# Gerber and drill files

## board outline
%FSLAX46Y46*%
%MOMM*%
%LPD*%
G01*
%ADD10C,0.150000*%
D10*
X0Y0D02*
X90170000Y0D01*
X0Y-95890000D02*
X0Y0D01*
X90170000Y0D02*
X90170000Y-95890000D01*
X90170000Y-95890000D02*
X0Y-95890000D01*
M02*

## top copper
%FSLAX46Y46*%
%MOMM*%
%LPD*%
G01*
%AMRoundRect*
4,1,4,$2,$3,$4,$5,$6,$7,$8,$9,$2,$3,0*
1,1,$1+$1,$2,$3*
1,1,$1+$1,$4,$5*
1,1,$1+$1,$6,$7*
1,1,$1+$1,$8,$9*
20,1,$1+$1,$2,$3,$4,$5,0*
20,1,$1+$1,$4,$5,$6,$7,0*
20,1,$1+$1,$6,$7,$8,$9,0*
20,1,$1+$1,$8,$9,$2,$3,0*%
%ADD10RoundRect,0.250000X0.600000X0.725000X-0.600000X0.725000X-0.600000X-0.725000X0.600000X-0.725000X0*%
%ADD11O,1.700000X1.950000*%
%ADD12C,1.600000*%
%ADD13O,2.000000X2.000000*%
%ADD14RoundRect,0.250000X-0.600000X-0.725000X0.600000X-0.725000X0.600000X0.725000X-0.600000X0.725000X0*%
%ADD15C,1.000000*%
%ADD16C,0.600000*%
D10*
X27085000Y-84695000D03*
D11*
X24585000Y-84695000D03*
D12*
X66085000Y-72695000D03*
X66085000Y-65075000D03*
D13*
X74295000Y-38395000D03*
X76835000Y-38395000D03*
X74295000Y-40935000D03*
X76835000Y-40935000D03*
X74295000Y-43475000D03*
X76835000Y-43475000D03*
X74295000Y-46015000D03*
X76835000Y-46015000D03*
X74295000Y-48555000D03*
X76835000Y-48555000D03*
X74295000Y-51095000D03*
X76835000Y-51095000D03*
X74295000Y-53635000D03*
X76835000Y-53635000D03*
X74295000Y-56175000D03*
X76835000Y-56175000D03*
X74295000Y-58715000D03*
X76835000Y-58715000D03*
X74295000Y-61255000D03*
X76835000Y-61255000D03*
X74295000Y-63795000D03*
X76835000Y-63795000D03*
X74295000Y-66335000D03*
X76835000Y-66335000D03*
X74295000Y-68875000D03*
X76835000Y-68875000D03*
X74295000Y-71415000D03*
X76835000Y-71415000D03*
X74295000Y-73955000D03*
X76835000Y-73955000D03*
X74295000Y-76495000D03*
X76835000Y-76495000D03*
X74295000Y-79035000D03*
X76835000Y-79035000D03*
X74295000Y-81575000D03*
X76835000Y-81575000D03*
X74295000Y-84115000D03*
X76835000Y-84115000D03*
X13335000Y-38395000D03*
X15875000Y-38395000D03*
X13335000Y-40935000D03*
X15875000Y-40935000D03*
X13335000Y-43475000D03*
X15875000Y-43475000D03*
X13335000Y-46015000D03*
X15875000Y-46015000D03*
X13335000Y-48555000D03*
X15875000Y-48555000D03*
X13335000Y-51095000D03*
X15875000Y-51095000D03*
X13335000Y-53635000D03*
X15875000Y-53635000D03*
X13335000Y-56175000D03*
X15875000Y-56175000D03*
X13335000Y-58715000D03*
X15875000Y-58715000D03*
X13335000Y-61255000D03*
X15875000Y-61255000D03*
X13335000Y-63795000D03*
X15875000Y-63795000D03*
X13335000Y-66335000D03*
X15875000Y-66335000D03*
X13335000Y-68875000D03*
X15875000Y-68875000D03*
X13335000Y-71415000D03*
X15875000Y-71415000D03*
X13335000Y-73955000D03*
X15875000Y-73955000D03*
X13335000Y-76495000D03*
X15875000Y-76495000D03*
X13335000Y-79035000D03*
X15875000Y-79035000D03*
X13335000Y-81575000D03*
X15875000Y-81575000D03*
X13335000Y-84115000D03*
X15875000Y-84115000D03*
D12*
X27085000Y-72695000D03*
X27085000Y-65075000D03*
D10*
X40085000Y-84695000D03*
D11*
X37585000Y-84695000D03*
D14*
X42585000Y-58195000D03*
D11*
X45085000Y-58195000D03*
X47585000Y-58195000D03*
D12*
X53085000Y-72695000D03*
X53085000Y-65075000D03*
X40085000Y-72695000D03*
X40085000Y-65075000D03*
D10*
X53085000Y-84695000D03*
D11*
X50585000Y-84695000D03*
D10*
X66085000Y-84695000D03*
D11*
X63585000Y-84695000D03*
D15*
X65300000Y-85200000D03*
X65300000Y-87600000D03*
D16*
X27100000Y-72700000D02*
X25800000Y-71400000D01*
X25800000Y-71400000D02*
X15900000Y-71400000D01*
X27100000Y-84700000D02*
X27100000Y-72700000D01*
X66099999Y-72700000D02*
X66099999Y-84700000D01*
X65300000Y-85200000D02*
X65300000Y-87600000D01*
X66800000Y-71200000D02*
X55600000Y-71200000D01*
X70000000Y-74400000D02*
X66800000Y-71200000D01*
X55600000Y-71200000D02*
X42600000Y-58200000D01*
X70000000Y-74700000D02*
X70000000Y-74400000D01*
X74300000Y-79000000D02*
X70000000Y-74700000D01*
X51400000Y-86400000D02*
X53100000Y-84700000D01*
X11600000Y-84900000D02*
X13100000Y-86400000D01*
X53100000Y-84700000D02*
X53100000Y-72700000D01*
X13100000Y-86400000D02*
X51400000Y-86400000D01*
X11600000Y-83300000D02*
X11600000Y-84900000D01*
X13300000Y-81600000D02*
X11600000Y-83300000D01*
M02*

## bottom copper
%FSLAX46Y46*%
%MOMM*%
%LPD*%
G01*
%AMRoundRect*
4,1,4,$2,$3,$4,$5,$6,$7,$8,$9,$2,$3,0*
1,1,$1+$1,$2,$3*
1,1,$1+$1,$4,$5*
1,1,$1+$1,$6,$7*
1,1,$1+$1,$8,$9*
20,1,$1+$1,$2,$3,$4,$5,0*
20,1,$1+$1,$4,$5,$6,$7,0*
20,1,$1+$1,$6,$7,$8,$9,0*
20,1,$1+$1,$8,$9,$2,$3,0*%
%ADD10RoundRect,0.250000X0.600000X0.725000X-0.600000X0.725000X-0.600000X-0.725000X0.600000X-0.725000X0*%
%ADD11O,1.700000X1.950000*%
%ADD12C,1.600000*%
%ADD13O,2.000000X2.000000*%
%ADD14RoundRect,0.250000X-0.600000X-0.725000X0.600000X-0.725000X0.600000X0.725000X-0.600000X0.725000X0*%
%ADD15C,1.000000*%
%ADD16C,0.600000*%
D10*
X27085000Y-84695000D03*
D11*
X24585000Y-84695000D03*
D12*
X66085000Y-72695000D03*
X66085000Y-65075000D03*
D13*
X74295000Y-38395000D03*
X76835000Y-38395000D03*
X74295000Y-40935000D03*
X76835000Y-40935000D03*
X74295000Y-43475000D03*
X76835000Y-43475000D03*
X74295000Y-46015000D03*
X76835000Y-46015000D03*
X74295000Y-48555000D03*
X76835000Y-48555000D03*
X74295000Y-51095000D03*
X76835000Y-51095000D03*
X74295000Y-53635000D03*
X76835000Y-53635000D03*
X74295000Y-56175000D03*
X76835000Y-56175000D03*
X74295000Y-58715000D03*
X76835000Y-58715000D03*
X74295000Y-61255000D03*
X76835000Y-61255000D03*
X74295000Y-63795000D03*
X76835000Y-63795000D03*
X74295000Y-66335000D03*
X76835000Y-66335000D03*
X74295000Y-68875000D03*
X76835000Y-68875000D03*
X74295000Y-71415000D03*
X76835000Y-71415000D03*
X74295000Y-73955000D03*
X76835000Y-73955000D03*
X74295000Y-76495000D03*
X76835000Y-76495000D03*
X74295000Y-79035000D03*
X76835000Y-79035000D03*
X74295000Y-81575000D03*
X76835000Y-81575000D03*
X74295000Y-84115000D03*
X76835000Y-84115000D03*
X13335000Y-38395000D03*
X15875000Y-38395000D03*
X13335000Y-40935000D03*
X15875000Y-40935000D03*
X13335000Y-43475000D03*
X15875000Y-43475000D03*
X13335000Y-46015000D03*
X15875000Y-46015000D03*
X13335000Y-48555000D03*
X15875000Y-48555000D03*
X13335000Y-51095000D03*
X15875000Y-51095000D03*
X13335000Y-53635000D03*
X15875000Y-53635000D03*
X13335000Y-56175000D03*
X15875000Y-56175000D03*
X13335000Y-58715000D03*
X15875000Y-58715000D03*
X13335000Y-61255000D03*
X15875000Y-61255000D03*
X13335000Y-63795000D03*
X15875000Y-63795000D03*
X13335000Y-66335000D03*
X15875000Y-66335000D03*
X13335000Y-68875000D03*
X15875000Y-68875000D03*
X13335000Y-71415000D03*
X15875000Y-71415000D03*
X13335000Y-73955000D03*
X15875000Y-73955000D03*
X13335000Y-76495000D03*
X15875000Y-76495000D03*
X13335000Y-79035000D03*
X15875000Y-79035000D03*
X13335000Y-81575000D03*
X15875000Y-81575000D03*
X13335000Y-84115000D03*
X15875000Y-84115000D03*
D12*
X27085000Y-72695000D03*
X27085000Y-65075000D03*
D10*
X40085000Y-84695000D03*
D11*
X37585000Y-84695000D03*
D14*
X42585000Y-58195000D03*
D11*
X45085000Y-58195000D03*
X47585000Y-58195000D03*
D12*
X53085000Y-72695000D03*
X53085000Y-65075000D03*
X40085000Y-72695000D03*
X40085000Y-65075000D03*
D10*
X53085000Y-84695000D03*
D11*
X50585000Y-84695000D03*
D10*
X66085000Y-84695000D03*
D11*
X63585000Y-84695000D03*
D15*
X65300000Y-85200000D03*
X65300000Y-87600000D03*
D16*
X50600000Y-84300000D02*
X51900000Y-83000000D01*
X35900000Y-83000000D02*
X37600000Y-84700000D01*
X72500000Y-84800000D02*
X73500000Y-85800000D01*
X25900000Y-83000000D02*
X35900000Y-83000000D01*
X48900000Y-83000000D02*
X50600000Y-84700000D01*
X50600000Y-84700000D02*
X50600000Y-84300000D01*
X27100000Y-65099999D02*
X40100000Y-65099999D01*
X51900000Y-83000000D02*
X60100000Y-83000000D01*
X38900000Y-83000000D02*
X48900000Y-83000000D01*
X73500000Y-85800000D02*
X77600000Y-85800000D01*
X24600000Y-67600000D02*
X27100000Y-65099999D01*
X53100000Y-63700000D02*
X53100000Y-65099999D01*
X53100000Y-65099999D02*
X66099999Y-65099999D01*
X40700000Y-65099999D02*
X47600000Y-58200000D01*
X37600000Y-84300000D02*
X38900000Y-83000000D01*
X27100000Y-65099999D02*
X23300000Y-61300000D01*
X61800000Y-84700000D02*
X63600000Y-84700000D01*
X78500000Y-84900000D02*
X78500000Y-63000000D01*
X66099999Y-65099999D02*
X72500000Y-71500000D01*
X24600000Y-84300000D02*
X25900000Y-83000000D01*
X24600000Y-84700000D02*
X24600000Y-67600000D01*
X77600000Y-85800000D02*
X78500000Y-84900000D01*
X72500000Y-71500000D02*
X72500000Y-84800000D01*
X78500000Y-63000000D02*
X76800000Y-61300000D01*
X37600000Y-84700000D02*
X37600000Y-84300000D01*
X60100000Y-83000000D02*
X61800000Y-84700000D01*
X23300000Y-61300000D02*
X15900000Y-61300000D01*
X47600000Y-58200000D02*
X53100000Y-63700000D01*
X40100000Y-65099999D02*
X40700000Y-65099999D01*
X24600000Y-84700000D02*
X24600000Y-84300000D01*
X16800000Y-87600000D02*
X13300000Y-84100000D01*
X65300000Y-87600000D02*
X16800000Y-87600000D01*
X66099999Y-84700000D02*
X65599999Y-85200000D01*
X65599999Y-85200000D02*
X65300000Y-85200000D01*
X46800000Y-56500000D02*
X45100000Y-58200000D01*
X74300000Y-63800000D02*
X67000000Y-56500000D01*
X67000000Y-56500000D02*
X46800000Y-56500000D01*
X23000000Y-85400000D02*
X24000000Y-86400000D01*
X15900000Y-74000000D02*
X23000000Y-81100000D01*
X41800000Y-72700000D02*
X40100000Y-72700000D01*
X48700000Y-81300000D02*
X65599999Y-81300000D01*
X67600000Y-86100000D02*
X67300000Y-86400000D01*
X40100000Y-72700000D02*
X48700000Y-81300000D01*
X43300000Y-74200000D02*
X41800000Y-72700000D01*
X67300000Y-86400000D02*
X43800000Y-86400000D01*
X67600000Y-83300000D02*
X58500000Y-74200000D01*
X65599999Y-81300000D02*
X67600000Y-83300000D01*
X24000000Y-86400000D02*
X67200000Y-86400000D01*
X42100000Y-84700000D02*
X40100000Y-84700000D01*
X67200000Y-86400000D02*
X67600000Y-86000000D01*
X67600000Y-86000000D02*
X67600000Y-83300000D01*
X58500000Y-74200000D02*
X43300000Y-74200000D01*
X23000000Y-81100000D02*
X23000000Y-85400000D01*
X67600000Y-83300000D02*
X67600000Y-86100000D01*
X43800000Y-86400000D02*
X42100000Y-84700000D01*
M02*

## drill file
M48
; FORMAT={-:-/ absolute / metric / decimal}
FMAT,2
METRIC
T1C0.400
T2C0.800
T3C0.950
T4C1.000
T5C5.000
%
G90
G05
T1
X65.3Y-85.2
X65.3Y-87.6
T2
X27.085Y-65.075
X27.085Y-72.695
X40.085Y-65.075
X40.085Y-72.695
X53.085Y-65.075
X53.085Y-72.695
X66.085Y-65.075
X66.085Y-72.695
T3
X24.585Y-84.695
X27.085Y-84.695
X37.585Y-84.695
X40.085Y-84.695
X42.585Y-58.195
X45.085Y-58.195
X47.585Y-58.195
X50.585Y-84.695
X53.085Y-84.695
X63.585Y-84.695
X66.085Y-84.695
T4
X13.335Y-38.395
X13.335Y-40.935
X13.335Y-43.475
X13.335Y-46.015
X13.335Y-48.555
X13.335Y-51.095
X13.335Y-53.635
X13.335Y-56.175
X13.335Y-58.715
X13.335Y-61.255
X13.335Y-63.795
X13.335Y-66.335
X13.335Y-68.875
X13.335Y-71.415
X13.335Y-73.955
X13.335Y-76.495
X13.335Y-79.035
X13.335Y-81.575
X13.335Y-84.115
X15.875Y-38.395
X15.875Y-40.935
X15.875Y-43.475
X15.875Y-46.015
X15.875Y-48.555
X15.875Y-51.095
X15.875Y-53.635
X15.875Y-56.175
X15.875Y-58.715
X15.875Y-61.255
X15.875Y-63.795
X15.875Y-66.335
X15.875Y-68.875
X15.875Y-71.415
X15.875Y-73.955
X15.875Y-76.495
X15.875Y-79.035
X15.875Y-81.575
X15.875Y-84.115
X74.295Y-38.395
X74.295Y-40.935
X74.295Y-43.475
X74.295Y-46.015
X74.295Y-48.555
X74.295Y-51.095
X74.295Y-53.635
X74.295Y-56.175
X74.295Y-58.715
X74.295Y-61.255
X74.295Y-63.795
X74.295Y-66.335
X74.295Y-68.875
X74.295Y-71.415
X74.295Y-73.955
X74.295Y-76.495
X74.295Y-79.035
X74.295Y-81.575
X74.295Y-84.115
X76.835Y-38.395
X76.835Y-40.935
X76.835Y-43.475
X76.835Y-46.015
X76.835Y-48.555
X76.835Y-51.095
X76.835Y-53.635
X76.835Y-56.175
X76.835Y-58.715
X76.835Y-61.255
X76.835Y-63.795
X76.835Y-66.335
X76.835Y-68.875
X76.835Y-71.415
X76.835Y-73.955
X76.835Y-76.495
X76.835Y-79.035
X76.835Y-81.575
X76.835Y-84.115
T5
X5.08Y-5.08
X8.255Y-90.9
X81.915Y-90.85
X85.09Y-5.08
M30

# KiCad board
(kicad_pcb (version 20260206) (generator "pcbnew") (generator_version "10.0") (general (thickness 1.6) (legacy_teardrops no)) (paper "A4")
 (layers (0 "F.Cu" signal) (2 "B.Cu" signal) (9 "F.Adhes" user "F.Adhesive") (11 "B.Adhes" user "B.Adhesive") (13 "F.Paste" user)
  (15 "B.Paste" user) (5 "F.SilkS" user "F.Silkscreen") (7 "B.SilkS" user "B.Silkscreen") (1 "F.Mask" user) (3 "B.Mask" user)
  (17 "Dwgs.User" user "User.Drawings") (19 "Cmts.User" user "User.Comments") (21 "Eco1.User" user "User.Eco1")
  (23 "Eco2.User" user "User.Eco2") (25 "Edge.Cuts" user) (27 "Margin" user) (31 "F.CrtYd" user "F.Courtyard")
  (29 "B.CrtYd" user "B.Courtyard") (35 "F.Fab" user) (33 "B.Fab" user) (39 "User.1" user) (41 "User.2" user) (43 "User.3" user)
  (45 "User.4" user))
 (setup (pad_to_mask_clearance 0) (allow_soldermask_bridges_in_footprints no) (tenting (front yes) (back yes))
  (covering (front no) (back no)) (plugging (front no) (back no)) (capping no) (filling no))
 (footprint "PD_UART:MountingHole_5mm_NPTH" (layer "F.Cu") (at 8.255 90.9)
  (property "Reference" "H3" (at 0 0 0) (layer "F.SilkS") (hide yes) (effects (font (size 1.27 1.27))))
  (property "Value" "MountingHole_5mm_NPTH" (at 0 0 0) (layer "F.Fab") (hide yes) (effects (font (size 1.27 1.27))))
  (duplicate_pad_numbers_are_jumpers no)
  (pad "" np_thru_hole circle (at 0 0) (size 5 5) (drill 5) (layers "*.Cu")))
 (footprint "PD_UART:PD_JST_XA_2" (layer "F.Cu") (at 27.085 84.695 180)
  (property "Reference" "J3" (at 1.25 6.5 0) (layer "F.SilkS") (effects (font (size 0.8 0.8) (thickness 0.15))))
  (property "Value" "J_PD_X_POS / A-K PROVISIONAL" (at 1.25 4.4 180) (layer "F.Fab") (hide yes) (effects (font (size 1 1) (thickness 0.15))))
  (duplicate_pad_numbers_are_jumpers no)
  (pad "1" thru_hole roundrect (at 0 0 180) (size 1.7 1.95) (drill 0.95) (layers "*.Cu") (remove_unused_layers no)
   (roundrect_rratio 0.147059) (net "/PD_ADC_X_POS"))
  (pad "2" thru_hole oval (at 2.5 0 180) (size 1.7 1.95) (drill 0.95) (layers "*.Cu") (remove_unused_layers no) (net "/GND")))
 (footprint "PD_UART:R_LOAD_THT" (layer "F.Cu") (at 66.085 72.695 90)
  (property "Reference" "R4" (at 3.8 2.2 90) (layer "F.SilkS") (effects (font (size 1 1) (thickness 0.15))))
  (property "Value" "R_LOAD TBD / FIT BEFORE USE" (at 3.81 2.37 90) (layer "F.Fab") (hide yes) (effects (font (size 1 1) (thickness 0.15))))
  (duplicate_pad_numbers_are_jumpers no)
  (pad "1" thru_hole circle (at 0 0 90) (size 1.6 1.6) (drill 0.8) (layers "*.Cu") (remove_unused_layers no) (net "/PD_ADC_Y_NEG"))
  (pad "2" thru_hole circle (at 7.62 0 90) (size 1.6 1.6) (drill 0.8) (layers "*.Cu") (remove_unused_layers no) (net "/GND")))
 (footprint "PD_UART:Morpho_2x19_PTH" (layer "F.Cu") (at 74.295 38.395)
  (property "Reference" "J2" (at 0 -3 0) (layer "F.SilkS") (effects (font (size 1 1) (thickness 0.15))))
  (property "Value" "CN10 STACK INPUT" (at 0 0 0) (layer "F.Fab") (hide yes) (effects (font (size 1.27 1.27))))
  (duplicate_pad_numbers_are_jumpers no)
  (pad "1" thru_hole oval (at 0 0) (size 2 2) (drill 1) (layers "*.Cu") (remove_unused_layers no) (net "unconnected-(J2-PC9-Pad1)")
   (thermal_bridge_angle 45))
  (pad "2" thru_hole oval (at 2.54 0) (size 2 2) (drill 1) (layers "*.Cu") (remove_unused_layers no) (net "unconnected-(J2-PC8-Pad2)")
   (thermal_bridge_angle 45))
  (pad "3" thru_hole oval (at 0 2.54) (size 2 2) (drill 1) (layers "*.Cu") (remove_unused_layers no) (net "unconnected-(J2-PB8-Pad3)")
   (thermal_bridge_angle 45))
  (pad "4" thru_hole oval (at 2.54 2.54) (size 2 2) (drill 1) (layers "*.Cu") (remove_unused_layers no) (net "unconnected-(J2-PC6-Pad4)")
   (thermal_bridge_angle 45))
  (pad "5" thru_hole oval (at 0 5.08) (size 2 2) (drill 1) (layers "*.Cu") (remove_unused_layers no) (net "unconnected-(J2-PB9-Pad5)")
   (thermal_bridge_angle 45))
  (pad "6" thru_hole oval (at 2.54 5.08) (size 2 2) (drill 1) (layers "*.Cu") (remove_unused_layers no) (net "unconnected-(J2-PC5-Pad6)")
   (thermal_bridge_angle 45))
  (pad "7" thru_hole oval (at 0 7.62) (size 2 2) (drill 1) (layers "*.Cu") (remove_unused_layers no) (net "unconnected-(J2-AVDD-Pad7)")
   (thermal_bridge_angle 45))
  (pad "8" thru_hole oval (at 2.54 7.62) (size 2 2) (drill 1) (layers "*.Cu") (remove_unused_layers no) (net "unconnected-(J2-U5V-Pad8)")
   (thermal_bridge_angle 45))
  (pad "9" thru_hole oval (at 0 10.16) (size 2 2) (drill 1) (layers "*.Cu") (remove_unused_layers no) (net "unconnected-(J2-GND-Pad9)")
   (thermal_bridge_angle 45))
  (pad "10" thru_hole oval (at 2.54 10.16) (size 2 2) (drill 1) (layers "*.Cu") (remove_unused_layers no) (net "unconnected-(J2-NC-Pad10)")
   (thermal_bridge_angle 45))
  (pad "11" thru_hole oval (at 0 12.7) (size 2 2) (drill 1) (layers "*.Cu") (remove_unused_layers no) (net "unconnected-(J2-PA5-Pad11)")
   (thermal_bridge_angle 45))
  (pad "12" thru_hole oval (at 2.54 12.7) (size 2 2) (drill 1) (layers "*.Cu") (remove_unused_layers no) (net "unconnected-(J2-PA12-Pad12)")
   (thermal_bridge_angle 45))
  (pad "13" thru_hole oval (at 0 15.24) (size 2 2) (drill 1) (layers "*.Cu") (remove_unused_layers no) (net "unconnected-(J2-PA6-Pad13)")
   (thermal_bridge_angle 45))
  (pad "14" thru_hole oval (at 2.54 15.24) (size 2 2) (drill 1) (layers "*.Cu") (remove_unused_layers no)
   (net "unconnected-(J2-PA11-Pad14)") (thermal_bridge_angle 45))
  (pad "15" thru_hole oval (at 0 17.78) (size 2 2) (drill 1) (layers "*.Cu") (remove_unused_layers no) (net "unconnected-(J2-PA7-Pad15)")
   (thermal_bridge_angle 45))
  (pad "16" thru_hole oval (at 2.54 17.78) (size 2 2) (drill 1) (layers "*.Cu") (remove_unused_layers no)
   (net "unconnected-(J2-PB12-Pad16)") (thermal_bridge_angle 45))
  (pad "17" thru_hole oval (at 0 20.32) (size 2 2) (drill 1) (layers "*.Cu") (remove_unused_layers no) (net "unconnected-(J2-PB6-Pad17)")
   (thermal_bridge_angle 45))
  (pad "18" thru_hole oval (at 2.54 20.32) (size 2 2) (drill 1) (layers "*.Cu") (remove_unused_layers no)
   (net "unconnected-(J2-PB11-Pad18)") (thermal_bridge_angle 45))
  (pad "19" thru_hole oval (at 0 22.86) (size 2 2) (drill 1) (layers "*.Cu") (remove_unused_layers no) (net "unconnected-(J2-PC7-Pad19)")
   (thermal_bridge_angle 45))
  (pad "20" thru_hole oval (at 2.54 22.86) (size 2 2) (drill 1) (layers "*.Cu") (remove_unused_layers no) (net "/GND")
   (thermal_bridge_angle 45))
  (pad "21" thru_hole oval (at 0 25.4) (size 2 2) (drill 1) (layers "*.Cu") (remove_unused_layers no) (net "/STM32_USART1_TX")
   (thermal_bridge_angle 45))
  (pad "22" thru_hole oval (at 2.54 25.4) (size 2 2) (drill 1) (layers "*.Cu") (remove_unused_layers no) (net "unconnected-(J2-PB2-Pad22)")
   (thermal_bridge_angle 45))
  (pad "23" thru_hole oval (at 0 27.94) (size 2 2) (drill 1) (layers "*.Cu") (remove_unused_layers no) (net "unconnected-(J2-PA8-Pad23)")
   (thermal_bridge_angle 45))
  (pad "24" thru_hole oval (at 2.54 27.94) (size 2 2) (drill 1) (layers "*.Cu") (remove_unused_layers no) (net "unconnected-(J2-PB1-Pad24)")
   (thermal_bridge_angle 45))
  (pad "25" thru_hole oval (at 0 30.48) (size 2 2) (drill 1) (layers "*.Cu") (remove_unused_layers no) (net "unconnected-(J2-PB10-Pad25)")
   (thermal_bridge_angle 45))
  (pad "26" thru_hole oval (at 2.54 30.48) (size 2 2) (drill 1) (layers "*.Cu") (remove_unused_layers no)
   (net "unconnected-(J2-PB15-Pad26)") (thermal_bridge_angle 45))
  (pad "27" thru_hole oval (at 0 33.02) (size 2 2) (drill 1) (layers "*.Cu") (remove_unused_layers no) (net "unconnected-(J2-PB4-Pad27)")
   (thermal_bridge_angle 45))
  (pad "28" thru_hole oval (at 2.54 33.02) (size 2 2) (drill 1) (layers "*.Cu") (remove_unused_layers no)
   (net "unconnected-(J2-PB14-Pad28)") (thermal_bridge_angle 45))
  (pad "29" thru_hole oval (at 0 35.56) (size 2 2) (drill 1) (layers "*.Cu") (remove_unused_layers no) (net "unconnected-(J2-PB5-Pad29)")
   (thermal_bridge_angle 45))
  (pad "30" thru_hole oval (at 2.54 35.56) (size 2 2) (drill 1) (layers "*.Cu") (remove_unused_layers no)
   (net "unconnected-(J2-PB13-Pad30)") (thermal_bridge_angle 45))
  (pad "31" thru_hole oval (at 0 38.1) (size 2 2) (drill 1) (layers "*.Cu") (remove_unused_layers no) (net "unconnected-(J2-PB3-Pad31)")
   (thermal_bridge_angle 45))
  (pad "32" thru_hole oval (at 2.54 38.1) (size 2 2) (drill 1) (layers "*.Cu") (remove_unused_layers no) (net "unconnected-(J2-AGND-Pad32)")
   (thermal_bridge_angle 45))
  (pad "33" thru_hole oval (at 0 40.64) (size 2 2) (drill 1) (layers "*.Cu") (remove_unused_layers no) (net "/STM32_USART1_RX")
   (thermal_bridge_angle 45))
  (pad "34" thru_hole oval (at 2.54 40.64) (size 2 2) (drill 1) (layers "*.Cu") (remove_unused_layers no) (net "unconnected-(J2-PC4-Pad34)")
   (thermal_bridge_angle 45))
  (pad "35" thru_hole oval (at 0 43.18) (size 2 2) (drill 1) (layers "*.Cu") (remove_unused_layers no) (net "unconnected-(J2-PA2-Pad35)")
   (thermal_bridge_angle 45))
  (pad "36" thru_hole oval (at 2.54 43.18) (size 2 2) (drill 1) (layers "*.Cu") (remove_unused_layers no) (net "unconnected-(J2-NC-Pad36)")
   (thermal_bridge_angle 45))
  (pad "37" thru_hole oval (at 0 45.72) (size 2 2) (drill 1) (layers "*.Cu") (remove_unused_layers no) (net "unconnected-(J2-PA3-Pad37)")
   (thermal_bridge_angle 45))
  (pad "38" thru_hole oval (at 2.54 45.72) (size 2 2) (drill 1) (layers "*.Cu") (remove_unused_layers no) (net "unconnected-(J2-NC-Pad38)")
   (thermal_bridge_angle 45)))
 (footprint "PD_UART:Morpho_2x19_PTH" (layer "F.Cu") (at 13.335 38.395)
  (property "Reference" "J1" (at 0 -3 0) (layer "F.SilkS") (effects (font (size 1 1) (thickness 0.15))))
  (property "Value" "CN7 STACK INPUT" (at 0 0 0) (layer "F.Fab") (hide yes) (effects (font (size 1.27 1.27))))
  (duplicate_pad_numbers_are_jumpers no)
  (pad "1" thru_hole oval (at 0 0) (size 2 2) (drill 1) (layers "*.Cu") (remove_unused_layers no) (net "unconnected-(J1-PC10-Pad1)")
   (thermal_bridge_angle 45))
  (pad "2" thru_hole oval (at 2.54 0) (size 2 2) (drill 1) (layers "*.Cu") (remove_unused_layers no) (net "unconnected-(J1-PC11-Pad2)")
   (thermal_bridge_angle 45))
  (pad "3" thru_hole oval (at 0 2.54) (size 2 2) (drill 1) (layers "*.Cu") (remove_unused_layers no) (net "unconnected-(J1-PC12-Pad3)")
   (thermal_bridge_angle 45))
  (pad "4" thru_hole oval (at 2.54 2.54) (size 2 2) (drill 1) (layers "*.Cu") (remove_unused_layers no) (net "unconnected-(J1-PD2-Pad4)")
   (thermal_bridge_angle 45))
  (pad "5" thru_hole oval (at 0 5.08) (size 2 2) (drill 1) (layers "*.Cu") (remove_unused_layers no) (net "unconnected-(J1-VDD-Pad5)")
   (thermal_bridge_angle 45))
  (pad "6" thru_hole oval (at 2.54 5.08) (size 2 2) (drill 1) (layers "*.Cu") (remove_unused_layers no) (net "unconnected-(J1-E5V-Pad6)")
   (thermal_bridge_angle 45))
  (pad "7" thru_hole oval (at 0 7.62) (size 2 2) (drill 1) (layers "*.Cu") (remove_unused_layers no) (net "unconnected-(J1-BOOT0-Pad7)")
   (thermal_bridge_angle 45))
  (pad "8" thru_hole oval (at 2.54 7.62) (size 2 2) (drill 1) (layers "*.Cu") (remove_unused_layers no) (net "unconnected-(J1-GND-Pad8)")
   (thermal_bridge_angle 45))
  (pad "9" thru_hole oval (at 0 10.16) (size 2 2) (drill 1) (layers "*.Cu") (remove_unused_layers no) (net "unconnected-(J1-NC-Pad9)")
   (thermal_bridge_angle 45))
  (pad "10" thru_hole oval (at 2.54 10.16) (size 2 2) (drill 1) (layers "*.Cu") (remove_unused_layers no) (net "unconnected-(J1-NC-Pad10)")
   (thermal_bridge_angle 45))
  (pad "11" thru_hole oval (at 0 12.7) (size 2 2) (drill 1) (layers "*.Cu") (remove_unused_layers no) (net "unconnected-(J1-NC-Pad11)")
   (thermal_bridge_angle 45))
  (pad "12" thru_hole oval (at 2.54 12.7) (size 2 2) (drill 1) (layers "*.Cu") (remove_unused_layers no)
   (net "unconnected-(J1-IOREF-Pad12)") (thermal_bridge_angle 45))
  (pad "13" thru_hole oval (at 0 15.24) (size 2 2) (drill 1) (layers "*.Cu") (remove_unused_layers no) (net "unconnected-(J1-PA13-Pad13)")
   (thermal_bridge_angle 45))
  (pad "14" thru_hole oval (at 2.54 15.24) (size 2 2) (drill 1) (layers "*.Cu") (remove_unused_layers no)
   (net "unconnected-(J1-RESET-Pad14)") (thermal_bridge_angle 45))
  (pad "15" thru_hole oval (at 0 17.78) (size 2 2) (drill 1) (layers "*.Cu") (remove_unused_layers no) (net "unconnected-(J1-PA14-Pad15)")
   (thermal_bridge_angle 45))
  (pad "16" thru_hole oval (at 2.54 17.78) (size 2 2) (drill 1) (layers "*.Cu") (remove_unused_layers no) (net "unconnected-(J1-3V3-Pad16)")
   (thermal_bridge_angle 45))
  (pad "17" thru_hole oval (at 0 20.32) (size 2 2) (drill 1) (layers "*.Cu") (remove_unused_layers no) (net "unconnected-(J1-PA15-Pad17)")
   (thermal_bridge_angle 45))
  (pad "18" thru_hole oval (at 2.54 20.32) (size 2 2) (drill 1) (layers "*.Cu") (remove_unused_layers no) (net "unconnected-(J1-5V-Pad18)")
   (thermal_bridge_angle 45))
  (pad "19" thru_hole oval (at 0 22.86) (size 2 2) (drill 1) (layers "*.Cu") (remove_unused_layers no) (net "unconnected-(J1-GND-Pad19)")
   (thermal_bridge_angle 45))
  (pad "20" thru_hole oval (at 2.54 22.86) (size 2 2) (drill 1) (layers "*.Cu") (remove_unused_layers no) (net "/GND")
   (thermal_bridge_angle 45))
  (pad "21" thru_hole oval (at 0 25.4) (size 2 2) (drill 1) (layers "*.Cu") (remove_unused_layers no) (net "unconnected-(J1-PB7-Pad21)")
   (thermal_bridge_angle 45))
  (pad "22" thru_hole oval (at 2.54 25.4) (size 2 2) (drill 1) (layers "*.Cu") (remove_unused_layers no) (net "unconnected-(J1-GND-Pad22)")
   (thermal_bridge_angle 45))
  (pad "23" thru_hole oval (at 0 27.94) (size 2 2) (drill 1) (layers "*.Cu") (remove_unused_layers no) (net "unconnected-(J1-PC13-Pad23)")
   (thermal_bridge_angle 45))
  (pad "24" thru_hole oval (at 2.54 27.94) (size 2 2) (drill 1) (layers "*.Cu") (remove_unused_layers no) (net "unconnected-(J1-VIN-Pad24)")
   (thermal_bridge_angle 45))
  (pad "25" thru_hole oval (at 0 30.48) (size 2 2) (drill 1) (layers "*.Cu") (remove_unused_layers no) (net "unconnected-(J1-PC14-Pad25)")
   (thermal_bridge_angle 45))
  (pad "26" thru_hole oval (at 2.54 30.48) (size 2 2) (drill 1) (layers "*.Cu") (remove_unused_layers no) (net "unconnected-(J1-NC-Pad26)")
   (thermal_bridge_angle 45))
  (pad "27" thru_hole oval (at 0 33.02) (size 2 2) (drill 1) (layers "*.Cu") (remove_unused_layers no) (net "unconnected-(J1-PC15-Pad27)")
   (thermal_bridge_angle 45))
  (pad "28" thru_hole oval (at 2.54 33.02) (size 2 2) (drill 1) (layers "*.Cu") (remove_unused_layers no) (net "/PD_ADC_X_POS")
   (thermal_bridge_angle 45))
  (pad "29" thru_hole oval (at 0 35.56) (size 2 2) (drill 1) (layers "*.Cu") (remove_unused_layers no) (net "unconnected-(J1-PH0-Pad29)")
   (thermal_bridge_angle 45))
  (pad "30" thru_hole oval (at 2.54 35.56) (size 2 2) (drill 1) (layers "*.Cu") (remove_unused_layers no) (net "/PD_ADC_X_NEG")
   (thermal_bridge_angle 45))
  (pad "31" thru_hole oval (at 0 38.1) (size 2 2) (drill 1) (layers "*.Cu") (remove_unused_layers no) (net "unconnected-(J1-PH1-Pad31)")
   (thermal_bridge_angle 45))
  (pad "32" thru_hole oval (at 2.54 38.1) (size 2 2) (drill 1) (layers "*.Cu") (remove_unused_layers no) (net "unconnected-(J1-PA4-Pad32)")
   (thermal_bridge_angle 45))
  (pad "33" thru_hole oval (at 0 40.64) (size 2 2) (drill 1) (layers "*.Cu") (remove_unused_layers no) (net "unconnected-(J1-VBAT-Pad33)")
   (thermal_bridge_angle 45))
  (pad "34" thru_hole oval (at 2.54 40.64) (size 2 2) (drill 1) (layers "*.Cu") (remove_unused_layers no) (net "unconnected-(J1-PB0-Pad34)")
   (thermal_bridge_angle 45))
  (pad "35" thru_hole oval (at 0 43.18) (size 2 2) (drill 1) (layers "*.Cu") (remove_unused_layers no) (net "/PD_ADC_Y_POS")
   (thermal_bridge_angle 45))
  (pad "36" thru_hole oval (at 2.54 43.18) (size 2 2) (drill 1) (layers "*.Cu") (remove_unused_layers no)
   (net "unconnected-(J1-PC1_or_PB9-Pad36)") (thermal_bridge_angle 45))
  (pad "37" thru_hole oval (at 0 45.72) (size 2 2) (drill 1) (layers "*.Cu") (remove_unused_layers no) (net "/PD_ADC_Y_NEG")
   (thermal_bridge_angle 45))
  (pad "38" thru_hole oval (at 2.54 45.72) (size 2 2) (drill 1) (layers "*.Cu") (remove_unused_layers no) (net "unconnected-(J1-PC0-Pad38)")
   (thermal_bridge_angle 45)))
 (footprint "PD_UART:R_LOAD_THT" (layer "F.Cu") (at 27.085 72.695 90)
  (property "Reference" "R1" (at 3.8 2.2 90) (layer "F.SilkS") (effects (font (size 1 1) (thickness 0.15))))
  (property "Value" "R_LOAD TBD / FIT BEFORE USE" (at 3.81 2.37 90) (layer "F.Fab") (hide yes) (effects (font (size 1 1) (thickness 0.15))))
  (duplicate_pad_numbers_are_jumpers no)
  (pad "1" thru_hole circle (at 0 0 90) (size 1.6 1.6) (drill 0.8) (layers "*.Cu") (remove_unused_layers no) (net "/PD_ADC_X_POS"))
  (pad "2" thru_hole circle (at 7.62 0 90) (size 1.6 1.6) (drill 0.8) (layers "*.Cu") (remove_unused_layers no) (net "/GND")))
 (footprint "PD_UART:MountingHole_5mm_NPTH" (layer "F.Cu") (at 81.915 90.85)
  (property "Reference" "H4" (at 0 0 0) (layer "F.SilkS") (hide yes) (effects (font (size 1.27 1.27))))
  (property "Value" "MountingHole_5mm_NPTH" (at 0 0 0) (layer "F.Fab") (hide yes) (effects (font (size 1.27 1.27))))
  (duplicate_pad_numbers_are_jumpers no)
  (pad "" np_thru_hole circle (at 0 0) (size 5 5) (drill 5) (layers "*.Cu")))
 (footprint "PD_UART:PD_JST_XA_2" (layer "F.Cu") (at 40.085 84.695 180)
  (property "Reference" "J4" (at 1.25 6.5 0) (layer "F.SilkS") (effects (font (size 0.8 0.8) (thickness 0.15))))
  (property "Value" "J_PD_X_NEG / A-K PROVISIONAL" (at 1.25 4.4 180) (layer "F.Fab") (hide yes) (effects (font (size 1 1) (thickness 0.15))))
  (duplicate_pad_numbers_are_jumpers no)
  (pad "1" thru_hole roundrect (at 0 0 180) (size 1.7 1.95) (drill 0.95) (layers "*.Cu") (remove_unused_layers no)
   (roundrect_rratio 0.147059) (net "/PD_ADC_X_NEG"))
  (pad "2" thru_hole oval (at 2.5 0 180) (size 1.7 1.95) (drill 0.95) (layers "*.Cu") (remove_unused_layers no) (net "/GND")))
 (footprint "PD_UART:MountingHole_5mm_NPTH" (layer "F.Cu") (at 85.09 5.08)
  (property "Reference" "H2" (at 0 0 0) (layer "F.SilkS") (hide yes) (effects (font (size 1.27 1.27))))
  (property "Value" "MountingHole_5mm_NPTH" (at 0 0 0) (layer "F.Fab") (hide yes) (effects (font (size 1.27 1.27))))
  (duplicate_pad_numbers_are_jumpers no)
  (pad "" np_thru_hole circle (at 0 0) (size 5 5) (drill 5) (layers "*.Cu")))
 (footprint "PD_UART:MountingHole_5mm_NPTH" (layer "F.Cu") (at 5.08 5.08)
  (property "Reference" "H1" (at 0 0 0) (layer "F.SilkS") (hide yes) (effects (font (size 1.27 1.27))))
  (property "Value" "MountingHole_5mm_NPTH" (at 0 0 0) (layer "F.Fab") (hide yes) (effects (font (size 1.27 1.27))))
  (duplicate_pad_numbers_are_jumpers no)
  (pad "" np_thru_hole circle (at 0 0) (size 5 5) (drill 5) (layers "*.Cu")))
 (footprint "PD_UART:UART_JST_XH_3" (layer "F.Cu") (at 42.585 58.195)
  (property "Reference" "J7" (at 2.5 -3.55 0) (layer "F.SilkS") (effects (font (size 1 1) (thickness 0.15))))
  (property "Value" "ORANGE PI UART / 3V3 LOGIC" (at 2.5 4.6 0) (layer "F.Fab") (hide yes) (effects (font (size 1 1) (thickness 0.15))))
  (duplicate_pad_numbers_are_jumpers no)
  (pad "1" thru_hole roundrect (at 0 0) (size 1.7 1.95) (drill 0.95) (layers "*.Cu") (remove_unused_layers no) (roundrect_rratio 0.147059)
   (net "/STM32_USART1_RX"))
  (pad "2" thru_hole oval (at 2.5 0) (size 1.7 1.95) (drill 0.95) (layers "*.Cu") (remove_unused_layers no) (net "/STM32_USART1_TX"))
  (pad "3" thru_hole oval (at 5 0) (size 1.7 1.95) (drill 0.95) (layers "*.Cu") (remove_unused_layers no) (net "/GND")))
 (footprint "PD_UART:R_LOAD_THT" (layer "F.Cu") (at 53.085 72.695 90)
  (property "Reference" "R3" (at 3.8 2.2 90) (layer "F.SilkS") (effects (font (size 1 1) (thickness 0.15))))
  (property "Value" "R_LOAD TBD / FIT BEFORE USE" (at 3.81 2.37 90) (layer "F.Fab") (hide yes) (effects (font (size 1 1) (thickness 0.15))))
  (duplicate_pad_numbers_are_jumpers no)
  (pad "1" thru_hole circle (at 0 0 90) (size 1.6 1.6) (drill 0.8) (layers "*.Cu") (remove_unused_layers no) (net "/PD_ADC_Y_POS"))
  (pad "2" thru_hole circle (at 7.62 0 90) (size 1.6 1.6) (drill 0.8) (layers "*.Cu") (remove_unused_layers no) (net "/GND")))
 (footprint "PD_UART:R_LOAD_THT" (layer "F.Cu") (at 40.085 72.695 90)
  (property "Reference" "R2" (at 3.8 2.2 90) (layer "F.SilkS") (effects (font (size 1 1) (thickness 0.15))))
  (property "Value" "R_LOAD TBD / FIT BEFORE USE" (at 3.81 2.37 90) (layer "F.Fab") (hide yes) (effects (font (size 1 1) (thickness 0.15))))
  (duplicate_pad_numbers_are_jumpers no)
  (pad "1" thru_hole circle (at 0 0 90) (size 1.6 1.6) (drill 0.8) (layers "*.Cu") (remove_unused_layers no) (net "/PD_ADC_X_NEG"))
  (pad "2" thru_hole circle (at 7.62 0 90) (size 1.6 1.6) (drill 0.8) (layers "*.Cu") (remove_unused_layers no) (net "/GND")))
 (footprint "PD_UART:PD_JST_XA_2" (layer "F.Cu") (at 53.085 84.695 180)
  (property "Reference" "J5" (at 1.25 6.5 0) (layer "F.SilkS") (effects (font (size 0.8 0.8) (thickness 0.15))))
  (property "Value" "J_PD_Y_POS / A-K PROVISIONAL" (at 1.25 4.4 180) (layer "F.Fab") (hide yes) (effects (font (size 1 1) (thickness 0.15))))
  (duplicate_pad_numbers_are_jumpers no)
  (pad "1" thru_hole roundrect (at 0 0 180) (size 1.7 1.95) (drill 0.95) (layers "*.Cu") (remove_unused_layers no)
   (roundrect_rratio 0.147059) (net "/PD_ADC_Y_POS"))
  (pad "2" thru_hole oval (at 2.5 0 180) (size 1.7 1.95) (drill 0.95) (layers "*.Cu") (remove_unused_layers no) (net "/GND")))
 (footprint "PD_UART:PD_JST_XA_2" (layer "F.Cu") (at 66.085 84.695 180)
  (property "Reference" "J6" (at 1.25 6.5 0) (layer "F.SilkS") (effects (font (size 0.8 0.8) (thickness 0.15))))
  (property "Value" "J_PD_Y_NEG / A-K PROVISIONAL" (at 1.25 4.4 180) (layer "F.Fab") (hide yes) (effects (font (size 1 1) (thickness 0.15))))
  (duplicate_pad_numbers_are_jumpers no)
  (pad "1" thru_hole roundrect (at 0 0 180) (size 1.7 1.95) (drill 0.95) (layers "*.Cu") (remove_unused_layers no)
   (roundrect_rratio 0.147059) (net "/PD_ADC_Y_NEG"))
  (pad "2" thru_hole oval (at 2.5 0 180) (size 1.7 1.95) (drill 0.95) (layers "*.Cu") (remove_unused_layers no) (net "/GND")))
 (gr_line (start 0 0) (end 90.17 0) (stroke (width 0.15) (type default)) (layer "Edge.Cuts"))
 (gr_line (start 0 95.89) (end 0 0) (stroke (width 0.15) (type default)) (layer "Edge.Cuts"))
 (gr_line (start 90.17 0) (end 90.17 95.89) (stroke (width 0.15) (type default)) (layer "Edge.Cuts"))
 (gr_line (start 90.17 95.89) (end 0 95.89) (stroke (width 0.15) (type default)) (layer "Edge.Cuts"))
 (segment (start 27.1 72.7) (end 25.8 71.4) (width 0.6) (layer "F.Cu") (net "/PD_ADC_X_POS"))
 (segment (start 25.8 71.4) (end 15.9 71.4) (width 0.6) (layer "F.Cu") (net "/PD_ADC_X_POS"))
 (segment (start 27.1 84.7) (end 27.1 72.7) (width 0.6) (layer "F.Cu") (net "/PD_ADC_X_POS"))
 (segment (start 50.6 84.3) (end 51.9 83) (width 0.6) (layer "B.Cu") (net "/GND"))
 (segment (start 35.9 83) (end 37.6 84.7) (width 0.6) (layer "B.Cu") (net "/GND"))
 (segment (start 72.5 84.8) (end 73.5 85.8) (width 0.6) (layer "B.Cu") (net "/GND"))
 (segment (start 25.9 83) (end 35.9 83) (width 0.6) (layer "B.Cu") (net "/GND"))
 (segment (start 48.9 83) (end 50.6 84.7) (width 0.6) (layer "B.Cu") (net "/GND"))
 (segment (start 50.6 84.7) (end 50.6 84.3) (width 0.6) (layer "B.Cu") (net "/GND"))
 (segment (start 27.1 65.099999) (end 40.1 65.099999) (width 0.6) (layer "B.Cu") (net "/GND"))
 (segment (start 51.9 83) (end 60.1 83) (width 0.6) (layer "B.Cu") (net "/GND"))
 (segment (start 38.9 83) (end 48.9 83) (width 0.6) (layer "B.Cu") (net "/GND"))
 (segment (start 73.5 85.8) (end 77.6 85.8) (width 0.6) (layer "B.Cu") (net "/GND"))
 (segment (start 24.6 67.6) (end 27.1 65.099999) (width 0.6) (layer "B.Cu") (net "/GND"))
 (segment (start 53.1 63.7) (end 53.1 65.099999) (width 0.6) (layer "B.Cu") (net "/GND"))
 (segment (start 53.1 65.099999) (end 66.099999 65.099999) (width 0.6) (layer "B.Cu") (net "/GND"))
 (segment (start 40.7 65.099999) (end 47.6 58.2) (width 0.6) (layer "B.Cu") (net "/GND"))
 (segment (start 37.6 84.3) (end 38.9 83) (width 0.6) (layer "B.Cu") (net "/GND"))
 (segment (start 27.1 65.099999) (end 23.3 61.3) (width 0.6) (layer "B.Cu") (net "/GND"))
 (segment (start 61.8 84.7) (end 63.6 84.7) (width 0.6) (layer "B.Cu") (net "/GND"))
 (segment (start 78.5 84.9) (end 78.5 63) (width 0.6) (layer "B.Cu") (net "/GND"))
 (segment (start 66.099999 65.099999) (end 72.5 71.5) (width 0.6) (layer "B.Cu") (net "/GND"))
 (segment (start 24.6 84.3) (end 25.9 83) (width 0.6) (layer "B.Cu") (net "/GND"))
 (segment (start 24.6 84.7) (end 24.6 67.6) (width 0.6) (layer "B.Cu") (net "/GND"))
 (segment (start 77.6 85.8) (end 78.5 84.9) (width 0.6) (layer "B.Cu") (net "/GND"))
 (segment (start 72.5 71.5) (end 72.5 84.8) (width 0.6) (layer "B.Cu") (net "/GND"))
 (segment (start 78.5 63) (end 76.8 61.3) (width 0.6) (layer "B.Cu") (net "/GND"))
 (segment (start 37.6 84.7) (end 37.6 84.3) (width 0.6) (layer "B.Cu") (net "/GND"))
 (segment (start 60.1 83) (end 61.8 84.7) (width 0.6) (layer "B.Cu") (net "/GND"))
 (segment (start 23.3 61.3) (end 15.9 61.3) (width 0.6) (layer "B.Cu") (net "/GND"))
 (segment (start 47.6 58.2) (end 53.1 63.7) (width 0.6) (layer "B.Cu") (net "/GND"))
 (segment (start 40.1 65.099999) (end 40.7 65.099999) (width 0.6) (layer "B.Cu") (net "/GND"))
 (segment (start 24.6 84.7) (end 24.6 84.3) (width 0.6) (layer "B.Cu") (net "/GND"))
 (segment (start 66.099999 72.7) (end 66.099999 84.7) (width 0.6) (layer "F.Cu") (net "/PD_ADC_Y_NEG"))
 (segment (start 65.3 85.2) (end 65.3 87.6) (width 0.6) (layer "F.Cu") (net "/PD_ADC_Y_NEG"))
 (via (at 65.3 85.2) (size 1) (drill 0.4) (layers "F.Cu" "B.Cu") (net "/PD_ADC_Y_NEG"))
 (via (at 65.3 87.6) (size 1) (drill 0.4) (layers "F.Cu" "B.Cu") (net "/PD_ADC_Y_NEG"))
 (segment (start 16.8 87.6) (end 13.3 84.1) (width 0.6) (layer "B.Cu") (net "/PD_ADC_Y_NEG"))
 (segment (start 65.3 87.6) (end 16.8 87.6) (width 0.6) (layer "B.Cu") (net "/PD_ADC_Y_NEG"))
 (segment (start 66.099999 84.7) (end 65.599999 85.2) (width 0.6) (layer "B.Cu") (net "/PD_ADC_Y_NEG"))
 (segment (start 65.599999 85.2) (end 65.3 85.2) (width 0.6) (layer "B.Cu") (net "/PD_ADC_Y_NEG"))
 (segment (start 46.8 56.5) (end 45.1 58.2) (width 0.6) (layer "B.Cu") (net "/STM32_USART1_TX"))
 (segment (start 74.3 63.8) (end 67 56.5) (width 0.6) (layer "B.Cu") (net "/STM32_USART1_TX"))
 (segment (start 67 56.5) (end 46.8 56.5) (width 0.6) (layer "B.Cu") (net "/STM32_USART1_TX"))
 (segment (start 66.8 71.2) (end 55.6 71.2) (width 0.6) (layer "F.Cu") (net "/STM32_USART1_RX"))
 (segment (start 70 74.4) (end 66.8 71.2) (width 0.6) (layer "F.Cu") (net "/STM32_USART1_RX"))
 (segment (start 55.6 71.2) (end 42.6 58.2) (width 0.6) (layer "F.Cu") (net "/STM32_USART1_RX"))
 (segment (start 70 74.7) (end 70 74.4) (width 0.6) (layer "F.Cu") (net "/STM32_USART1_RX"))
 (segment (start 74.3 79) (end 70 74.7) (width 0.6) (layer "F.Cu") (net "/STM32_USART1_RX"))
 (segment (start 23 85.4) (end 24 86.4) (width 0.6) (layer "B.Cu") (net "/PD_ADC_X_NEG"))
 (segment (start 15.9 74) (end 23 81.1) (width 0.6) (layer "B.Cu") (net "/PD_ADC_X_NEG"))
 (segment (start 41.8 72.7) (end 40.1 72.7) (width 0.6) (layer "B.Cu") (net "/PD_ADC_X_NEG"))
 (segment (start 48.7 81.3) (end 65.599999 81.3) (width 0.6) (layer "B.Cu") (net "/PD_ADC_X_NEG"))
 (segment (start 67.6 86.1) (end 67.3 86.4) (width 0.6) (layer "B.Cu") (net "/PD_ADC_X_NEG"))
 (segment (start 40.1 72.7) (end 48.7 81.3) (width 0.6) (layer "B.Cu") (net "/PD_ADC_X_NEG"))
 (segment (start 43.3 74.2) (end 41.8 72.7) (width 0.6) (layer "B.Cu") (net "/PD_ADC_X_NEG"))
 (segment (start 67.3 86.4) (end 43.8 86.4) (width 0.6) (layer "B.Cu") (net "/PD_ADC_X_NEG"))
 (segment (start 67.6 83.3) (end 58.5 74.2) (width 0.6) (layer "B.Cu") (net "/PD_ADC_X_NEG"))
 (segment (start 65.599999 81.3) (end 67.6 83.3) (width 0.6) (layer "B.Cu") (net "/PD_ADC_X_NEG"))
 (segment (start 24 86.4) (end 67.2 86.4) (width 0.6) (layer "B.Cu") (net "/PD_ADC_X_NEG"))
 (segment (start 42.1 84.7) (end 40.1 84.7) (width 0.6) (layer "B.Cu") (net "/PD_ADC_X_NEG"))
 (segment (start 67.2 86.4) (end 67.6 86) (width 0.6) (layer "B.Cu") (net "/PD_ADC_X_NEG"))
 (segment (start 67.6 86) (end 67.6 83.3) (width 0.6) (layer "B.Cu") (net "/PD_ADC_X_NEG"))
 (segment (start 58.5 74.2) (end 43.3 74.2) (width 0.6) (layer "B.Cu") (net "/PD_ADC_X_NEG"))
 (segment (start 23 81.1) (end 23 85.4) (width 0.6) (layer "B.Cu") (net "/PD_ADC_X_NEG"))
 (segment (start 67.6 83.3) (end 67.6 86.1) (width 0.6) (layer "B.Cu") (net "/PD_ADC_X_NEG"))
 (segment (start 43.8 86.4) (end 42.1 84.7) (width 0.6) (layer "B.Cu") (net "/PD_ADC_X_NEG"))
 (segment (start 51.4 86.4) (end 53.1 84.7) (width 0.6) (layer "F.Cu") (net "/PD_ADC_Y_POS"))
 (segment (start 11.6 84.9) (end 13.1 86.4) (width 0.6) (layer "F.Cu") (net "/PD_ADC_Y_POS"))
 (segment (start 53.1 84.7) (end 53.1 72.7) (width 0.6) (layer "F.Cu") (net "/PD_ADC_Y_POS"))
 (segment (start 13.1 86.4) (end 51.4 86.4) (width 0.6) (layer "F.Cu") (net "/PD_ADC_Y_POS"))
 (segment (start 11.6 83.3) (end 11.6 84.9) (width 0.6) (layer "F.Cu") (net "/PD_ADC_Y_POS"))
 (segment (start 13.3 81.6) (end 11.6 83.3) (width 0.6) (layer "F.Cu") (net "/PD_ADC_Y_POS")))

